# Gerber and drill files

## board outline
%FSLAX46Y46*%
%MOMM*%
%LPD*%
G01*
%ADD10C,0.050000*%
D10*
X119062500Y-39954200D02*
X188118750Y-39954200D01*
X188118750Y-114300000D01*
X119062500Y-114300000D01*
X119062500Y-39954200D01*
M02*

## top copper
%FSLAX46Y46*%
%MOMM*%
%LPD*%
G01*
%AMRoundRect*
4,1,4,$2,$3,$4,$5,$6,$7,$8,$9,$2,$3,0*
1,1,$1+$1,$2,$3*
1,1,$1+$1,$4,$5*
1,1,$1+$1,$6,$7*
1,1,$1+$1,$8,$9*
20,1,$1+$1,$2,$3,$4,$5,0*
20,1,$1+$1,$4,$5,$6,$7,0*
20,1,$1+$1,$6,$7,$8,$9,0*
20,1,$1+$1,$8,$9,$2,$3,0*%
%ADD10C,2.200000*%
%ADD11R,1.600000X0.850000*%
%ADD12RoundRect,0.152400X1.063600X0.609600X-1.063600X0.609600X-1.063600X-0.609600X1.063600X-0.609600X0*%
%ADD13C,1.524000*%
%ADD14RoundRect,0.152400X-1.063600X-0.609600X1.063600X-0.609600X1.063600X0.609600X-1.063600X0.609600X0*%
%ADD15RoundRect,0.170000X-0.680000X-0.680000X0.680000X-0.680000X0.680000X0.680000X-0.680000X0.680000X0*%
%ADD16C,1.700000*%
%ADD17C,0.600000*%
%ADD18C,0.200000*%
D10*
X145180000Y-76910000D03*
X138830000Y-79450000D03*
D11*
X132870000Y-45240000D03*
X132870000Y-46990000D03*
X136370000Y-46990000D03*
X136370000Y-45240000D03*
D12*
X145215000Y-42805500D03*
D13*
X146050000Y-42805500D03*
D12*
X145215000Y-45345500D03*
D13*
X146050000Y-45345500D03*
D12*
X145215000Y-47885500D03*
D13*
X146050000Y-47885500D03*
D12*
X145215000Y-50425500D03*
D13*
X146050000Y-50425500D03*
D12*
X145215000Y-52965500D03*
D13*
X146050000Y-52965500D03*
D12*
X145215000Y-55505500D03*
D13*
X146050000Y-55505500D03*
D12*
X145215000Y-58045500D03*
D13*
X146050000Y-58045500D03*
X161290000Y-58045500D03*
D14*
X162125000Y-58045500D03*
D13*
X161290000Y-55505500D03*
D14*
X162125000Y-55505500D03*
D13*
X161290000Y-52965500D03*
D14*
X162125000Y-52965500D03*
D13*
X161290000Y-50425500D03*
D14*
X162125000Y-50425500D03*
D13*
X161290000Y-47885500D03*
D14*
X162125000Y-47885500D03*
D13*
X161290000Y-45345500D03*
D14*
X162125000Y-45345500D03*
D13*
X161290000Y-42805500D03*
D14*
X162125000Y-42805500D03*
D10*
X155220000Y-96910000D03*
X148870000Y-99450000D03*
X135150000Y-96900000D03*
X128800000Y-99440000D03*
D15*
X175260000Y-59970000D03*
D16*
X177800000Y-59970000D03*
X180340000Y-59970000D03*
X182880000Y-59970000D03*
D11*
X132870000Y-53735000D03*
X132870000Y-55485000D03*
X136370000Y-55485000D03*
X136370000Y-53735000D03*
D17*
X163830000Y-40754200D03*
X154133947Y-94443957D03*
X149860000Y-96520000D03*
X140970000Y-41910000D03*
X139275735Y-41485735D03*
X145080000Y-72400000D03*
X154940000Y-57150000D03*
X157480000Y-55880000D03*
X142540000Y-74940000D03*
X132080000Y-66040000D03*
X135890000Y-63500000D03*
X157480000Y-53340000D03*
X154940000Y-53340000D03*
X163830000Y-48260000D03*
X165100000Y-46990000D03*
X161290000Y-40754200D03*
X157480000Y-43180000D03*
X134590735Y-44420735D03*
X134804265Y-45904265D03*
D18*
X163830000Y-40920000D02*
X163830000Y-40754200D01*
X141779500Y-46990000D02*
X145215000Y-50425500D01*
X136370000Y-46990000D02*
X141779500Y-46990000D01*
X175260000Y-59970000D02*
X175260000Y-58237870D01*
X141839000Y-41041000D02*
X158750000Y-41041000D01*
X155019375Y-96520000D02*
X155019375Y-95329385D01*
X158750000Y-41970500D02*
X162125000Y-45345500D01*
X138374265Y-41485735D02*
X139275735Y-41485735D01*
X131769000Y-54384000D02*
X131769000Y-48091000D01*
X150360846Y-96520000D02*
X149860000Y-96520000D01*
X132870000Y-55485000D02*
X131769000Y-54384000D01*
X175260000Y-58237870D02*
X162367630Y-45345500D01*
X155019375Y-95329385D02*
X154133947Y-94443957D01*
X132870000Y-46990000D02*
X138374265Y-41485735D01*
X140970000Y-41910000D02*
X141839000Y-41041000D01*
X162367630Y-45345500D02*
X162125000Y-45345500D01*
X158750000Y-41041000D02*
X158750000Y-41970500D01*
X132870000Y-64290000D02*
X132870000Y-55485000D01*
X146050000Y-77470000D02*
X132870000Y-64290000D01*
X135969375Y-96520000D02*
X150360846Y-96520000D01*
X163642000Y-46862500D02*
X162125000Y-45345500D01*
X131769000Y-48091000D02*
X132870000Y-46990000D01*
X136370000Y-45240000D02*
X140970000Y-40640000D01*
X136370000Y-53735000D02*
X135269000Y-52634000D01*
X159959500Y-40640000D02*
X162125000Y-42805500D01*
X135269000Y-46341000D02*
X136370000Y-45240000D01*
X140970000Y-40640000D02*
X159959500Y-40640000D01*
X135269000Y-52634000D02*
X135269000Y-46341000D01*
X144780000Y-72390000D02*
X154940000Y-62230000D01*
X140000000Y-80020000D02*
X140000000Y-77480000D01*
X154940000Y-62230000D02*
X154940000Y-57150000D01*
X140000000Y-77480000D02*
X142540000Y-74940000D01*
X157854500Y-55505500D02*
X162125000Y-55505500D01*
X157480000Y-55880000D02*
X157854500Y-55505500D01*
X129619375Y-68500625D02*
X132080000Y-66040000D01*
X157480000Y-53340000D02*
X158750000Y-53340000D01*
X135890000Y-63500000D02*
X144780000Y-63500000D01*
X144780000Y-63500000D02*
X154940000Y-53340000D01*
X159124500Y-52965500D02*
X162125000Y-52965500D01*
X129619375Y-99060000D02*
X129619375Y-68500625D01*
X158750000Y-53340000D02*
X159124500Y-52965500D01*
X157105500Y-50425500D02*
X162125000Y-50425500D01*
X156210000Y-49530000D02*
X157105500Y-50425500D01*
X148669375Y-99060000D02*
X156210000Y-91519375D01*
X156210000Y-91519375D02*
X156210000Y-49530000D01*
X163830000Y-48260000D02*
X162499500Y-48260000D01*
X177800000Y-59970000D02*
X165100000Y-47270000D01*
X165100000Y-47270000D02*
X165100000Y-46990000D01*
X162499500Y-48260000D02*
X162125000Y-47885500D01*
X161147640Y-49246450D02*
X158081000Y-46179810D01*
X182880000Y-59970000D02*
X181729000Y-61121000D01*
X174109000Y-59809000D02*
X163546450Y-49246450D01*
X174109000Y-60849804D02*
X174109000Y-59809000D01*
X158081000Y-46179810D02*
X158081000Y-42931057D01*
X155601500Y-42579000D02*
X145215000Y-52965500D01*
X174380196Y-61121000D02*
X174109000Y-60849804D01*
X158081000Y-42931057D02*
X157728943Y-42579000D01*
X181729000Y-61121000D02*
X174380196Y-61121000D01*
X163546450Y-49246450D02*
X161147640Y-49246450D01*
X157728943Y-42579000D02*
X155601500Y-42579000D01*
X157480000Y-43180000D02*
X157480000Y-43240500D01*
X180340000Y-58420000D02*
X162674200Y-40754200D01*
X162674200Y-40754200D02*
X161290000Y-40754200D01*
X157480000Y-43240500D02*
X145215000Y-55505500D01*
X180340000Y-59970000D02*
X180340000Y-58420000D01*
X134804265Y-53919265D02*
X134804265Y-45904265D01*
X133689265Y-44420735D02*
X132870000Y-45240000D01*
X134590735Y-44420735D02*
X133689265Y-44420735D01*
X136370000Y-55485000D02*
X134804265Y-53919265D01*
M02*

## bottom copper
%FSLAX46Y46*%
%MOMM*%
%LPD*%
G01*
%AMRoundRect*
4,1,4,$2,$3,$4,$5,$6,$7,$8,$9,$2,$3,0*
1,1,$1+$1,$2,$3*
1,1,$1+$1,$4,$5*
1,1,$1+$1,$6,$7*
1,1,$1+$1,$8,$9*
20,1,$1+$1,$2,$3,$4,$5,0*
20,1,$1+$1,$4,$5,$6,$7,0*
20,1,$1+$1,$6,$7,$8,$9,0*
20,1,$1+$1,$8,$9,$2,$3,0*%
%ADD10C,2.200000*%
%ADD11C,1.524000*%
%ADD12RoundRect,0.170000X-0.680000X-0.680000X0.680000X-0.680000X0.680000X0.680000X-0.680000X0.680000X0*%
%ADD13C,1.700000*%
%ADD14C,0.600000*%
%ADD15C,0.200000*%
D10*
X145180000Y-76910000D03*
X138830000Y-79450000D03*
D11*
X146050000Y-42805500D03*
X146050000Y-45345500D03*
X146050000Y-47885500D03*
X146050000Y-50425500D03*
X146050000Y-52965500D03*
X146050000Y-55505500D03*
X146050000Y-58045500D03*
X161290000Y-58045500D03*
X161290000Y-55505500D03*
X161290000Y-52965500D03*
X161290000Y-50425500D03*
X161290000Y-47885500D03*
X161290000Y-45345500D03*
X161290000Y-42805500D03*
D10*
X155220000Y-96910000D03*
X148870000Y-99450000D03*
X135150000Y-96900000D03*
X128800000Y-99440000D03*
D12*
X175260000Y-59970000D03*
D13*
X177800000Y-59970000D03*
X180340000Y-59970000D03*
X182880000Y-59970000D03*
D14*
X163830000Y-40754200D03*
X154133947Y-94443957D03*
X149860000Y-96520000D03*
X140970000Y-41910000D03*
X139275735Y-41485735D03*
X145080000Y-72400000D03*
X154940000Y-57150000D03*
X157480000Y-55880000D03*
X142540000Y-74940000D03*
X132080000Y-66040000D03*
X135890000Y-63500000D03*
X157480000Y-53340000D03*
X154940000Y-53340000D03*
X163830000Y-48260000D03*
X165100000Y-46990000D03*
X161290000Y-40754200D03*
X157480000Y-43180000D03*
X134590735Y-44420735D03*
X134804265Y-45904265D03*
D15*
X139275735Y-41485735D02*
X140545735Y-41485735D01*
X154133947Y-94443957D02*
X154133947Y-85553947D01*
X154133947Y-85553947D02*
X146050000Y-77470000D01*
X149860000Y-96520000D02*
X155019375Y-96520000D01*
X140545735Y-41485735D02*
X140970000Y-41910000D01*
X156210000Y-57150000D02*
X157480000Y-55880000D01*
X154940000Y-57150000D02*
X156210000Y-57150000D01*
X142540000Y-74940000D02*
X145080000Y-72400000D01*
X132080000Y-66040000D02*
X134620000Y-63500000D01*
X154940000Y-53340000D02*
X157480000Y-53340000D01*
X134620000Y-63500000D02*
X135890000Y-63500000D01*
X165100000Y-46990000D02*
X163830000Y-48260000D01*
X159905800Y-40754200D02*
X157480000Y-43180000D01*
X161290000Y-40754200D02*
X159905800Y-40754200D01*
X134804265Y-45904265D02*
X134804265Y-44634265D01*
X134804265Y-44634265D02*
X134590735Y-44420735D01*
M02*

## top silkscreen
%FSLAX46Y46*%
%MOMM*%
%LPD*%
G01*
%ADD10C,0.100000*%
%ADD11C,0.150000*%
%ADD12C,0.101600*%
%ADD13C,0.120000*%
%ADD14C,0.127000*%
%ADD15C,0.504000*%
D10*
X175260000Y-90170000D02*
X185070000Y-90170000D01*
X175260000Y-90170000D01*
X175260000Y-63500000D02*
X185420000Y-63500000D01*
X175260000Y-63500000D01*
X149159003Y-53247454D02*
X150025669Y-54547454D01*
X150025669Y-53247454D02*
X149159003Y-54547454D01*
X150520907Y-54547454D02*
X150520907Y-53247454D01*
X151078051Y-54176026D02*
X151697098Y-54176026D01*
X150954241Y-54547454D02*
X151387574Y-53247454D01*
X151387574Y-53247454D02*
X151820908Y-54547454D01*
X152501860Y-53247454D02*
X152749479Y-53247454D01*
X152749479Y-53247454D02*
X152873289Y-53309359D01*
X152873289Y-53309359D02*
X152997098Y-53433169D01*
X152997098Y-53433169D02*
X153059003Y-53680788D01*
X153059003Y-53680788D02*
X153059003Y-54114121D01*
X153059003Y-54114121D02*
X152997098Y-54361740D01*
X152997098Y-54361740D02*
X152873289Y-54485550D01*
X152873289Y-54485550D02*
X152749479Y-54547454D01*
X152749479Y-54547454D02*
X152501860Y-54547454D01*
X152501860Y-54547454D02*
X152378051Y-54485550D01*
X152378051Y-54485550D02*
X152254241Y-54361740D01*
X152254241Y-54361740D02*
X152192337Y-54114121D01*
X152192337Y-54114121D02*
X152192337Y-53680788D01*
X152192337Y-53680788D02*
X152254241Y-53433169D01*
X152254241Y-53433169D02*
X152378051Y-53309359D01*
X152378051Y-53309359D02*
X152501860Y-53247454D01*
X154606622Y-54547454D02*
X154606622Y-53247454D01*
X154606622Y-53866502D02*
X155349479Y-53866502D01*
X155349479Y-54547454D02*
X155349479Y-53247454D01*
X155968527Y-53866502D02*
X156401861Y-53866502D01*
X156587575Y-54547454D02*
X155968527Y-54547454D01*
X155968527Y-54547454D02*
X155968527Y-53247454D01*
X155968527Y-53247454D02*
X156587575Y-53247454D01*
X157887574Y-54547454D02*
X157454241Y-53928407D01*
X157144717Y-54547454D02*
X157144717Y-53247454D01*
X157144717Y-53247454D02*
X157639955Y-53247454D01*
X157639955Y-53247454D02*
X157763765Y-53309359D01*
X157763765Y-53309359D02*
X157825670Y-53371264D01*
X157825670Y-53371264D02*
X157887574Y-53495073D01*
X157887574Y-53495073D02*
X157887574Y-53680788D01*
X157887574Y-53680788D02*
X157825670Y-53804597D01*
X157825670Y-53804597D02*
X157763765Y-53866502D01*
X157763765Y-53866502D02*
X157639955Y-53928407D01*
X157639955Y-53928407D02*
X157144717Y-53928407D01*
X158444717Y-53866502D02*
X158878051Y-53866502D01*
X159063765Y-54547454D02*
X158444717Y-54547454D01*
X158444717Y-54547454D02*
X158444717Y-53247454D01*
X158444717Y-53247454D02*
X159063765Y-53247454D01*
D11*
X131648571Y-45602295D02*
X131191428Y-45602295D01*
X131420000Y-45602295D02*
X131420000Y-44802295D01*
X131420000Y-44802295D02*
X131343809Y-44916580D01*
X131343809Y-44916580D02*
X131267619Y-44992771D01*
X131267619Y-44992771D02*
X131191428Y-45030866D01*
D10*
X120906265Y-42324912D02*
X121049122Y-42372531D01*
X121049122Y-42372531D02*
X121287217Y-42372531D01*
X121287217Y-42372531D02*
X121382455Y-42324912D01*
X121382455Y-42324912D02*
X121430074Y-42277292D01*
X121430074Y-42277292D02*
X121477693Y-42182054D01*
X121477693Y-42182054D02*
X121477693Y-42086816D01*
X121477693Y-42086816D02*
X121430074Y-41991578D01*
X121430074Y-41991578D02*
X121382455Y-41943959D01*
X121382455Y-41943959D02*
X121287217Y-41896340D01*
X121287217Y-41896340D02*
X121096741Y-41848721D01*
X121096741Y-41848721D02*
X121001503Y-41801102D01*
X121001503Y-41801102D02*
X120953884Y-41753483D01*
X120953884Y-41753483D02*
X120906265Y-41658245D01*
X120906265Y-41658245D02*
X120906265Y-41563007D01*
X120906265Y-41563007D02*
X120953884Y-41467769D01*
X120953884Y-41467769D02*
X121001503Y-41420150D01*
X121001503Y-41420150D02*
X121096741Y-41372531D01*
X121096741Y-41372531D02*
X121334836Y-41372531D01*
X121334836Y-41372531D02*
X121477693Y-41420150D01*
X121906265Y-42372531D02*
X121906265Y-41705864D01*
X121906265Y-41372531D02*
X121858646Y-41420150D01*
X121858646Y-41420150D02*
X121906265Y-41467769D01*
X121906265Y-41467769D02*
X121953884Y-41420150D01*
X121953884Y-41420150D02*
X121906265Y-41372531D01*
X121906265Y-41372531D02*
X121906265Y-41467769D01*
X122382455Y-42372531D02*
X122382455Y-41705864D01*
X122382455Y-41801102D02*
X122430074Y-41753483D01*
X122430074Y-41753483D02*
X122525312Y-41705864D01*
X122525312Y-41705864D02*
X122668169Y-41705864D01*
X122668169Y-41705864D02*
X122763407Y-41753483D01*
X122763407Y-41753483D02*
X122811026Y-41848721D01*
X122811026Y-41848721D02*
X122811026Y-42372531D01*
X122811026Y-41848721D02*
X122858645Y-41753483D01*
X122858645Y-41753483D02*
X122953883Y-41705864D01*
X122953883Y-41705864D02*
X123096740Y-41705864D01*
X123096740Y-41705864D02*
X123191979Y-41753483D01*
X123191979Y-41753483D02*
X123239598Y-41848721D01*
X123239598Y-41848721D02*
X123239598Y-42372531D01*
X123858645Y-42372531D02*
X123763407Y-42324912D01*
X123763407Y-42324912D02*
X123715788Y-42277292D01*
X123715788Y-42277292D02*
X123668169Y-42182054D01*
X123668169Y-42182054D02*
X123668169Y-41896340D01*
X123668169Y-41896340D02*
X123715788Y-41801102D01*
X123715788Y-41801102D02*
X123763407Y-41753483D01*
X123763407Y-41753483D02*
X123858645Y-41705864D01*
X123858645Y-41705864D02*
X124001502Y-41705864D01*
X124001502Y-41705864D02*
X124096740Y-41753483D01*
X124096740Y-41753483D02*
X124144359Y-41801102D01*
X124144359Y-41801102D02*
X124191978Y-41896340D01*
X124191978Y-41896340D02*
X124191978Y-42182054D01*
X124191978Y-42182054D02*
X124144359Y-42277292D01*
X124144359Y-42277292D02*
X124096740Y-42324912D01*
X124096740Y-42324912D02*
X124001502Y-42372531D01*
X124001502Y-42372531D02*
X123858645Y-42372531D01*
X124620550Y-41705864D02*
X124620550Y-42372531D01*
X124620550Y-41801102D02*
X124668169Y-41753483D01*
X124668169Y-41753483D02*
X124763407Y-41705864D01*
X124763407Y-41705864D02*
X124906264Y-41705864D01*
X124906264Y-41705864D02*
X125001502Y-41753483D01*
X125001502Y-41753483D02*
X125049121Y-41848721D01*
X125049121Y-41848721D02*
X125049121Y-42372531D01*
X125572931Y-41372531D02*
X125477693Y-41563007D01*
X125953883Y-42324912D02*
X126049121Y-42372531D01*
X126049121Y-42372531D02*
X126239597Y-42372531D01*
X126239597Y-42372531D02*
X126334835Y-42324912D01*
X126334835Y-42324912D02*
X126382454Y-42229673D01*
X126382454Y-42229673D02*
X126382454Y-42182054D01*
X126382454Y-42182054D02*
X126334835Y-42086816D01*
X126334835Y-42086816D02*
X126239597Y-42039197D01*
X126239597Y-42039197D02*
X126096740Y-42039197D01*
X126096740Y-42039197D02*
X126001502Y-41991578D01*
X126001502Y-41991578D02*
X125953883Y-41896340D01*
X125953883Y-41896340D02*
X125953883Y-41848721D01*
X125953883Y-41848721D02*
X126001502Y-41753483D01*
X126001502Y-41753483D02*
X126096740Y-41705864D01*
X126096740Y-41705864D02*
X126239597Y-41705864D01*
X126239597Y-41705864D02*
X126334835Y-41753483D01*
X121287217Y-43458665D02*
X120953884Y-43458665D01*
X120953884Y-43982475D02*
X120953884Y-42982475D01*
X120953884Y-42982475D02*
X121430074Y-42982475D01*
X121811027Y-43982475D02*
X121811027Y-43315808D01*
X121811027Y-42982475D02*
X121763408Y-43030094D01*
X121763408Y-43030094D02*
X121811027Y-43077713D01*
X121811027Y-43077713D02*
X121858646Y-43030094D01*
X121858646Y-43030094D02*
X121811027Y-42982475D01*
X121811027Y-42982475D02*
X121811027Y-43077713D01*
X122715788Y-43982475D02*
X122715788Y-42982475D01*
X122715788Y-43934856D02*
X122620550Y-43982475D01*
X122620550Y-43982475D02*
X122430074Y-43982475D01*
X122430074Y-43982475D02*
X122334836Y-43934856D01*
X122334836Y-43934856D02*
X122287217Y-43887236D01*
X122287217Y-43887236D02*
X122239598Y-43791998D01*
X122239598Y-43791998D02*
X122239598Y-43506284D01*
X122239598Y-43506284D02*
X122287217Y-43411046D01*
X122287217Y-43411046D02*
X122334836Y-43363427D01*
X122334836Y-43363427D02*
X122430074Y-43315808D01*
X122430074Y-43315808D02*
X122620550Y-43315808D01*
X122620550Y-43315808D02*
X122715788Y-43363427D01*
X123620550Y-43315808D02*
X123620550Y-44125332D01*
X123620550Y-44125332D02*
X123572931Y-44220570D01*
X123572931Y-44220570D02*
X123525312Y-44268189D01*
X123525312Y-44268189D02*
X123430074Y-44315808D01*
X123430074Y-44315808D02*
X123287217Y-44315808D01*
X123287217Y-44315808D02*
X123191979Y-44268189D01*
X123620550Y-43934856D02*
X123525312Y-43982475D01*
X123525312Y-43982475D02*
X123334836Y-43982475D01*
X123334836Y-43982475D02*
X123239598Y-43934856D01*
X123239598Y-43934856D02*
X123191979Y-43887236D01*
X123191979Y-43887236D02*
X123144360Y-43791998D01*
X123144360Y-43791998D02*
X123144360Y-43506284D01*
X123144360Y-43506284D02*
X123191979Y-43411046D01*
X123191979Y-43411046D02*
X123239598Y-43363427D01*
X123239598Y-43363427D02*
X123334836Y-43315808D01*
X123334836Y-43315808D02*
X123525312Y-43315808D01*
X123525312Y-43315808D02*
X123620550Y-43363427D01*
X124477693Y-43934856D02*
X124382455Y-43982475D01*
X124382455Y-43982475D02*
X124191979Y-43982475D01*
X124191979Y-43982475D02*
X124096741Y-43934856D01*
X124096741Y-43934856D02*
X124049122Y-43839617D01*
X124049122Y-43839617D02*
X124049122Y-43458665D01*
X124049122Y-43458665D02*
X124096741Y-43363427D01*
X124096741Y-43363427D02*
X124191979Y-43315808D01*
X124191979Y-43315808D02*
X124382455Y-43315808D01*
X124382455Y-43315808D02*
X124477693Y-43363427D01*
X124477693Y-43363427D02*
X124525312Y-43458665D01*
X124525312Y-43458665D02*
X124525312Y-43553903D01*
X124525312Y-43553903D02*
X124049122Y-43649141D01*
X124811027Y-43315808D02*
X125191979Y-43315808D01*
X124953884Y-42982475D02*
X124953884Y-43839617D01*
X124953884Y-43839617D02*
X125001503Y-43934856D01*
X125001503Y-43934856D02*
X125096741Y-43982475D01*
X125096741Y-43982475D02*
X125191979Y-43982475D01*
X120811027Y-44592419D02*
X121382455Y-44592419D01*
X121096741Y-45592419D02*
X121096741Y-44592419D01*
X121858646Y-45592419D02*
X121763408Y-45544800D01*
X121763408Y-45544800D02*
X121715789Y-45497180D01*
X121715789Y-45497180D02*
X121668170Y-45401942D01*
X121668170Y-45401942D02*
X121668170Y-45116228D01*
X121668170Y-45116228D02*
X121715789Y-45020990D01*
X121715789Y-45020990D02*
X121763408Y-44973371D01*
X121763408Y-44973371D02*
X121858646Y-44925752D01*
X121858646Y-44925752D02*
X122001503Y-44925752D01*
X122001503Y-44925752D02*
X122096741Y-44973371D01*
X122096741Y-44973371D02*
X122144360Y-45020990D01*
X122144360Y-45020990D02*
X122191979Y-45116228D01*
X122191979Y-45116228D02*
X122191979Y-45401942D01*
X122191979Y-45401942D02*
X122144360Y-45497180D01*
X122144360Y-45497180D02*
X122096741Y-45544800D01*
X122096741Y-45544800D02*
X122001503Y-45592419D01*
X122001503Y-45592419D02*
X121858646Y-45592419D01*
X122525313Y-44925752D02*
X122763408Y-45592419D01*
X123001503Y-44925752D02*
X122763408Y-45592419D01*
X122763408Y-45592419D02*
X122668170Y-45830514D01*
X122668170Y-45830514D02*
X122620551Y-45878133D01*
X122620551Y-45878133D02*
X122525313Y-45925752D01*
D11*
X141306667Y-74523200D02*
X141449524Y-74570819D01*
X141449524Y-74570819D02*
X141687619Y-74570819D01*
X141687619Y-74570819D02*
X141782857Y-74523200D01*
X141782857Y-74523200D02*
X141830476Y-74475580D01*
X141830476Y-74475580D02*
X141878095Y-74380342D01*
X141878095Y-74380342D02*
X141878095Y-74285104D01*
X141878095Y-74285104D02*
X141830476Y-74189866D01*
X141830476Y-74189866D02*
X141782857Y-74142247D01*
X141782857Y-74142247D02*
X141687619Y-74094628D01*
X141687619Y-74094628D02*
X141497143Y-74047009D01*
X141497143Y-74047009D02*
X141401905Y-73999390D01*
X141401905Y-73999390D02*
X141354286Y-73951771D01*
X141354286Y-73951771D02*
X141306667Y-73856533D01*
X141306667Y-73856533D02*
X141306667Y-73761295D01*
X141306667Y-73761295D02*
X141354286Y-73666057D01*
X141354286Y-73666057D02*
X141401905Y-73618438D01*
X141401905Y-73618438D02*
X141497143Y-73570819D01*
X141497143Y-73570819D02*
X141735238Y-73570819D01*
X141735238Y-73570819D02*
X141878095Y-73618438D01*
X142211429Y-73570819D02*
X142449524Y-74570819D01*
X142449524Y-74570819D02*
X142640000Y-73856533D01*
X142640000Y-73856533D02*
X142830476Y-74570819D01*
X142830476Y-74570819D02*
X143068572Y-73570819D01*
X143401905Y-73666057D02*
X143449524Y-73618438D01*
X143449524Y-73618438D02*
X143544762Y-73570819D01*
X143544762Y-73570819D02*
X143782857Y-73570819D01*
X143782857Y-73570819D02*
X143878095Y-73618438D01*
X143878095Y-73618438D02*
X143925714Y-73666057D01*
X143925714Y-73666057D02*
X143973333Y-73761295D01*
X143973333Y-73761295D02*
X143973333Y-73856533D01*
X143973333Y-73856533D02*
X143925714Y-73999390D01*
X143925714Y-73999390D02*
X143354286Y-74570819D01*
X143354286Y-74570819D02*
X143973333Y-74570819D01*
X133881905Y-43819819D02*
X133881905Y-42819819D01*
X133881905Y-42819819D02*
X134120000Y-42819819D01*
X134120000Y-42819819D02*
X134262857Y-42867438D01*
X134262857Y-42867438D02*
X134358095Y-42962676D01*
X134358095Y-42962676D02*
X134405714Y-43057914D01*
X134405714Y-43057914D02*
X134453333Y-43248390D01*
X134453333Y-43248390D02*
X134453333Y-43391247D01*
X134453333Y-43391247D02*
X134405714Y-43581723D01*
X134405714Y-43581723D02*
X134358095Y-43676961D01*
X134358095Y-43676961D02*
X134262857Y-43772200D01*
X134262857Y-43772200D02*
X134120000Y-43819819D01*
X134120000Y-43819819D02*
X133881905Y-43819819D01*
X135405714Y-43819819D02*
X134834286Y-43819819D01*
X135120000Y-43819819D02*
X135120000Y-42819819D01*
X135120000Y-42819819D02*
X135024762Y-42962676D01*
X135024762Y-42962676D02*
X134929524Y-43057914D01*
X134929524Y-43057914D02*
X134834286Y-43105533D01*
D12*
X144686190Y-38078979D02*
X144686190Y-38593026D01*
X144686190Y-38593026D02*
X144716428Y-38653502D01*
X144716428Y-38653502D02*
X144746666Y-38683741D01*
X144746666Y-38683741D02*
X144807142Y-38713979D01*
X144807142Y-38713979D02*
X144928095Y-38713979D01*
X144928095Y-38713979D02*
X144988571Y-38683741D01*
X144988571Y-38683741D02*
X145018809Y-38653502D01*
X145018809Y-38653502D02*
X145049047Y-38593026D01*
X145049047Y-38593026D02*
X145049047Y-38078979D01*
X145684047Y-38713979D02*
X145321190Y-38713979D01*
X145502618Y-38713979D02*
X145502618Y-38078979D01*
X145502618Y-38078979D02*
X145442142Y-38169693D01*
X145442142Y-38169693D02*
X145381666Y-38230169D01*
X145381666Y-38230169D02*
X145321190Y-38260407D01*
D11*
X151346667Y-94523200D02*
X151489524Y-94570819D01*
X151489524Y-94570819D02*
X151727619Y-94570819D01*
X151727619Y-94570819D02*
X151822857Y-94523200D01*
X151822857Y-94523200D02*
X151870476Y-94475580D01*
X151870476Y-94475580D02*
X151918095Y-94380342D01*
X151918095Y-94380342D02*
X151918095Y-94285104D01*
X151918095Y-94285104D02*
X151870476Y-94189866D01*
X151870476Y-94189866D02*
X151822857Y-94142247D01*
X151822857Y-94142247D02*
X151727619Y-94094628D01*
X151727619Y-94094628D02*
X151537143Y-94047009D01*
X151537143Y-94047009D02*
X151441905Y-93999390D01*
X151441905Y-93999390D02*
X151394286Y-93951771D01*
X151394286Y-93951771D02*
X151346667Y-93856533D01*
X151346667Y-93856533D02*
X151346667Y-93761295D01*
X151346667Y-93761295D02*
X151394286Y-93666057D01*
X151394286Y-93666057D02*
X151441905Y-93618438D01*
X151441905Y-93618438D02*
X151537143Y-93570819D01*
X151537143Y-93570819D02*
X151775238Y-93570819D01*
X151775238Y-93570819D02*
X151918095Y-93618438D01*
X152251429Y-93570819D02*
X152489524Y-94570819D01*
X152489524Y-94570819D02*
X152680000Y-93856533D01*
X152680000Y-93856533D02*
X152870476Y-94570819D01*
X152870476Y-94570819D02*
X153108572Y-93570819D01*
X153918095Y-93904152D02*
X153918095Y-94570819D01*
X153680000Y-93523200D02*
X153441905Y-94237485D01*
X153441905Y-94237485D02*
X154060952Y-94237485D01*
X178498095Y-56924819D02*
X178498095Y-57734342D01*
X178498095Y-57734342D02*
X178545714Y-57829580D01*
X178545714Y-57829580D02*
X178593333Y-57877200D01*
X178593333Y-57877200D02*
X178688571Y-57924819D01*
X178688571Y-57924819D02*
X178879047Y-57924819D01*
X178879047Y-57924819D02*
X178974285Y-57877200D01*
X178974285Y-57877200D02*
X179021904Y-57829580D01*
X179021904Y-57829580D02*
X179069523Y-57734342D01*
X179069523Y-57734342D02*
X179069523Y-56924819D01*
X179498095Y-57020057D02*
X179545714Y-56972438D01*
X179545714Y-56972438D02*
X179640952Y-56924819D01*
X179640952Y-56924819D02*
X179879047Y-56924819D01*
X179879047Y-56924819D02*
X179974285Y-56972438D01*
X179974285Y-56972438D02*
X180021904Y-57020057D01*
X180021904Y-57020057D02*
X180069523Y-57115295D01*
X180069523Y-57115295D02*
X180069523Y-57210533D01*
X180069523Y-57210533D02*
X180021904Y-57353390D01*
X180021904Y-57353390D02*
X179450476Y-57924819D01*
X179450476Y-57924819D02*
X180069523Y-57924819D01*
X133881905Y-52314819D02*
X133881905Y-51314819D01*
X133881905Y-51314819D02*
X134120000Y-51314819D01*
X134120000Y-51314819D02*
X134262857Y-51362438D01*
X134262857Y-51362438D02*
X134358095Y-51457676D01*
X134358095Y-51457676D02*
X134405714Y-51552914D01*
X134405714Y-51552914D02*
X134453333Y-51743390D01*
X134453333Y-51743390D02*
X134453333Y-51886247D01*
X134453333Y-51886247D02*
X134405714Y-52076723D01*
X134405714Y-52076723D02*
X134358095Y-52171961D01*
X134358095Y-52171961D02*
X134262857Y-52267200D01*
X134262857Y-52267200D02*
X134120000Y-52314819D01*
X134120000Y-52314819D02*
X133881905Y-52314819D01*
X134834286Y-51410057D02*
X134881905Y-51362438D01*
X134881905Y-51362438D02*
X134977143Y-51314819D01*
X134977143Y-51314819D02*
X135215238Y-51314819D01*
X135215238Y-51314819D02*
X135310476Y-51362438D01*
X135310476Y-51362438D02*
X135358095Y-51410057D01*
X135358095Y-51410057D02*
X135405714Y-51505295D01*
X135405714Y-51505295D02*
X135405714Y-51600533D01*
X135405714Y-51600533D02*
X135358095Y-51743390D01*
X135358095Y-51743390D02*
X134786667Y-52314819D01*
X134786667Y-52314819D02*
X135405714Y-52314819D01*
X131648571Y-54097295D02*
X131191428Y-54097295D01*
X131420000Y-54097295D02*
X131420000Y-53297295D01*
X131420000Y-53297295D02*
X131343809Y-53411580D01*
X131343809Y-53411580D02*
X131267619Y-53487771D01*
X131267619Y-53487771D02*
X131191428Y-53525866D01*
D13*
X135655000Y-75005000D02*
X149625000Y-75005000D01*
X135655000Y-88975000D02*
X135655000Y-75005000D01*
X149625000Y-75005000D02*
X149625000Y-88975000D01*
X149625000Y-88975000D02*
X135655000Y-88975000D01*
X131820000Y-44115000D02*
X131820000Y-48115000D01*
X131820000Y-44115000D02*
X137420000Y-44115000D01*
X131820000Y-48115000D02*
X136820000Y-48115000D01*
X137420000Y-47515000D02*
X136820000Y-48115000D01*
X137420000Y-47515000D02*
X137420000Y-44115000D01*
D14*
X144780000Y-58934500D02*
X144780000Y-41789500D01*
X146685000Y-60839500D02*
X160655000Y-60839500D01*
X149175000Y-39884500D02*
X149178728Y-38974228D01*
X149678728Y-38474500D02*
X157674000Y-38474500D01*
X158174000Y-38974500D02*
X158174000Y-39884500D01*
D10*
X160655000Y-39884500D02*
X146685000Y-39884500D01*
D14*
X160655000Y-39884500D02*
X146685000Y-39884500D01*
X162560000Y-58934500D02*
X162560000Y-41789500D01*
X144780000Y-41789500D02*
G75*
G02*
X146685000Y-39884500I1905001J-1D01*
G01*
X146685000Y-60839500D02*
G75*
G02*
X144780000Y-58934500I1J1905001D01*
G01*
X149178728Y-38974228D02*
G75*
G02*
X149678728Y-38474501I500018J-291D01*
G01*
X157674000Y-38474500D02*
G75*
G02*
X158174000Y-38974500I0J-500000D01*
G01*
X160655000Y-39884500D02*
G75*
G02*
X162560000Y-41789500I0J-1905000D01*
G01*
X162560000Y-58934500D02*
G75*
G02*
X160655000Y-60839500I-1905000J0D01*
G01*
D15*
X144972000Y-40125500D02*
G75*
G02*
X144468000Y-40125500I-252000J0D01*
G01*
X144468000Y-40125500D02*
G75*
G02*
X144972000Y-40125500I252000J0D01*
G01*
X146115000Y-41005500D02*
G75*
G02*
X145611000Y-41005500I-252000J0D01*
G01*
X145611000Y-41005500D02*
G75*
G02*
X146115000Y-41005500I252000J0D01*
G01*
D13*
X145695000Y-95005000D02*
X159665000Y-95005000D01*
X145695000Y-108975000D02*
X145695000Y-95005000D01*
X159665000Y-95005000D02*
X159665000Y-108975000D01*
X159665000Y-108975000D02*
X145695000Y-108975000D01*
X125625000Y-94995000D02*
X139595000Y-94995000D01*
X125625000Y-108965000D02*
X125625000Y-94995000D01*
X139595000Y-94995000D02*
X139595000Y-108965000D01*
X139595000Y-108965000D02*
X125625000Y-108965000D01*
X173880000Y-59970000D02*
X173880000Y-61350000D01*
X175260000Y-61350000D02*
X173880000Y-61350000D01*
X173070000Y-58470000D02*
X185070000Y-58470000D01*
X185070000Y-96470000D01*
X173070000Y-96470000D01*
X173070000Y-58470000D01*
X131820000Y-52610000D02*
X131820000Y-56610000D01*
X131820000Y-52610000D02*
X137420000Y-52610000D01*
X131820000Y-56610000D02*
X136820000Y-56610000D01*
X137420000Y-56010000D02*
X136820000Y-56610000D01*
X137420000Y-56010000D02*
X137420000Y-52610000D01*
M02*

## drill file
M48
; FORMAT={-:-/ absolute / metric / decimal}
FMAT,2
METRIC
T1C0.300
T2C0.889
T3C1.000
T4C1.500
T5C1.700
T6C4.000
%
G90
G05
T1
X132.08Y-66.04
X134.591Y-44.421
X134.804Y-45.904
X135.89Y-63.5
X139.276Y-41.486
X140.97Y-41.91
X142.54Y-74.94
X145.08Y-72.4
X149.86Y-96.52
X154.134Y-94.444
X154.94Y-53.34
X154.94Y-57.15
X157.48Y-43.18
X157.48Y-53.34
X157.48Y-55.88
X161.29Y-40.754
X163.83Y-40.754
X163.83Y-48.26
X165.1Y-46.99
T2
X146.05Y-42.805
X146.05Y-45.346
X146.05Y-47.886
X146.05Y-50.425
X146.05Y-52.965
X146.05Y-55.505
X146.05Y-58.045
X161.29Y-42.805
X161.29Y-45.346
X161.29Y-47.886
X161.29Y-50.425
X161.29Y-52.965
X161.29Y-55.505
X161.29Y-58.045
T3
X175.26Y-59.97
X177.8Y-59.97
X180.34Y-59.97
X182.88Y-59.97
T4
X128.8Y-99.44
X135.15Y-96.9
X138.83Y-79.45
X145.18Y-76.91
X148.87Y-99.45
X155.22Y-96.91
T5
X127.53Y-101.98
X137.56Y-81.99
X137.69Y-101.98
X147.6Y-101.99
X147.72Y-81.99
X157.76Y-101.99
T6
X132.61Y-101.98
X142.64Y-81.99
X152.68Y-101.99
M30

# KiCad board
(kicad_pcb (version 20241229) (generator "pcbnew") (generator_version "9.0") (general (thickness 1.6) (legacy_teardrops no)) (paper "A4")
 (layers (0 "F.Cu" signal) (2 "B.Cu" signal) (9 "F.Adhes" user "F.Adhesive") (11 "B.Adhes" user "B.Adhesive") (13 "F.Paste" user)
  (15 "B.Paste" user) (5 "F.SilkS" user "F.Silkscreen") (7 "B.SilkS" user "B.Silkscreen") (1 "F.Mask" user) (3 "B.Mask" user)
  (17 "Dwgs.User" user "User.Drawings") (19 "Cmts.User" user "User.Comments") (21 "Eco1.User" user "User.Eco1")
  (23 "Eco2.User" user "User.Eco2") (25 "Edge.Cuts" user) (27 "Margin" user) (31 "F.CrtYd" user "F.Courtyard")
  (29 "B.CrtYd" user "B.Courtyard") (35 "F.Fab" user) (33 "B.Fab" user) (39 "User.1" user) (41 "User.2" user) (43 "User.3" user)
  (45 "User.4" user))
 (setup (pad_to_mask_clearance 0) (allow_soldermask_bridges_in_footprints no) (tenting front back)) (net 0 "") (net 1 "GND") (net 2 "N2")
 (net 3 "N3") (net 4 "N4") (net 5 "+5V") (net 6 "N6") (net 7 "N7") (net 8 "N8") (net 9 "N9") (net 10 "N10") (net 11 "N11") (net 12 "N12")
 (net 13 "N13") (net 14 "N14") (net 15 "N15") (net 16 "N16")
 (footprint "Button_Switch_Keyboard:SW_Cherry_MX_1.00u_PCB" (layer "F.Cu") (at 145.18 76.91)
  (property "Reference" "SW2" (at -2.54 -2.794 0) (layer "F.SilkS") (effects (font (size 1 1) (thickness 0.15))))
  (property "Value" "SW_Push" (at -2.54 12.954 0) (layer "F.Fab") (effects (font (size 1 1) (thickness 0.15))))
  (fp_line (start -9.525 -1.905) (end 4.445 -1.905) (stroke (width 0.12) (type solid)) (layer "F.SilkS"))
  (fp_line (start -9.525 12.065) (end -9.525 -1.905) (stroke (width 0.12) (type solid)) (layer "F.SilkS"))
  (fp_line (start 4.445 -1.905) (end 4.445 12.065) (stroke (width 0.12) (type solid)) (layer "F.SilkS"))
  (fp_line (start 4.445 12.065) (end -9.525 12.065) (stroke (width 0.12) (type solid)) (layer "F.SilkS"))
  (pad "" np_thru_hole circle (at -7.62 5.08) (size 1.7 1.7) (drill 1.7) (layers "*.Cu" "*.Mask"))
  (pad "" np_thru_hole circle (at -2.54 5.08) (size 4 4) (drill 4) (layers "*.Cu" "*.Mask"))
  (pad "" np_thru_hole circle (at 2.54 5.08) (size 1.7 1.7) (drill 1.7) (layers "*.Cu" "*.Mask"))
  (pad "1" thru_hole circle (at 0 0) (size 2.2 2.2) (drill 1.5) (layers "*.Cu" "*.Mask") (remove_unused_layers no) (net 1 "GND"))
  (pad "2" thru_hole circle (at -6.35 2.54) (size 2.2 2.2) (drill 1.5) (layers "*.Cu" "*.Mask") (remove_unused_layers no) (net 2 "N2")))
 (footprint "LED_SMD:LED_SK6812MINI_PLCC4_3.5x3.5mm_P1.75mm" (layer "F.Cu") (at 134.62 46.115)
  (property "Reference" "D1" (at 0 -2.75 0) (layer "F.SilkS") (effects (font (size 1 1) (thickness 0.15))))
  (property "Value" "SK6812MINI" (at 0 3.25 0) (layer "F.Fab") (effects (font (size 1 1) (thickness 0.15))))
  (fp_line (start -2.8 -2) (end -2.8 2) (stroke (width 0.12) (type default)) (layer "F.SilkS"))
  (fp_line (start -2.8 -2) (end 2.8 -2) (stroke (width 0.12) (type solid)) (layer "F.SilkS"))
  (fp_line (start -2.8 2) (end 2.2 2) (stroke (width 0.12) (type solid)) (layer "F.SilkS"))
  (fp_line (start 2.8 1.4) (end 2.2 2) (stroke (width 0.12) (type default)) (layer "F.SilkS"))
  (fp_line (start 2.8 1.4) (end 2.8 -2) (stroke (width 0.12) (type solid)) (layer "F.SilkS"))
  (pad "1" smd rect (at -1.75 -0.875) (size 1.6 0.85) (layers "F.Cu" "F.Mask" "F.Paste") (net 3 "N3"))
  (pad "2" smd rect (at -1.75 0.875) (size 1.6 0.85) (layers "F.Cu" "F.Mask" "F.Paste") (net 1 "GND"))
  (pad "3" smd rect (at 1.75 0.875) (size 1.6 0.85) (layers "F.Cu" "F.Mask" "F.Paste") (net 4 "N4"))
  (pad "4" smd rect (at 1.75 -0.875) (size 1.6 0.85) (layers "F.Cu" "F.Mask" "F.Paste") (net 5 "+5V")))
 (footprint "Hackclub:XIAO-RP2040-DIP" (layer "F.Cu") (at 153.67 50.4255)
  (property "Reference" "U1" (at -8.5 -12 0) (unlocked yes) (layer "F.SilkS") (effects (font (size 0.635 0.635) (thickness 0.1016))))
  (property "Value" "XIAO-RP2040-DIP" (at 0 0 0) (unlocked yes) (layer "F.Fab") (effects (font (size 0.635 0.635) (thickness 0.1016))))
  (fp_line (start -8.89 8.509) (end -8.89 -8.636) (stroke (width 0.127) (type solid)) (layer "F.SilkS"))
  (fp_line (start -6.985 10.414) (end 6.985 10.414) (stroke (width 0.127) (type solid)) (layer "F.SilkS"))
  (fp_line (start -4.495 -10.541) (end -4.491272 -11.451272) (stroke (width 0.127) (type solid)) (layer "F.SilkS"))
  (fp_line (start -3.991272 -11.951) (end 4.004 -11.951) (stroke (width 0.127) (type solid)) (layer "F.SilkS"))
  (fp_line (start 4.504 -11.451) (end 4.504 -10.541) (stroke (width 0.127) (type solid)) (layer "F.SilkS"))
  (fp_line (start 6.985 -10.541) (end -6.985 -10.541) (stroke (width 0.1) (type solid)) (layer "F.SilkS"))
  (fp_line (start 6.985 -10.541) (end -6.985 -10.541) (stroke (width 0.127) (type solid)) (layer "F.SilkS"))
  (fp_line (start 8.89 8.509) (end 8.89 -8.636) (stroke (width 0.127) (type solid)) (layer "F.SilkS"))
  (fp_arc (start -8.89 -8.636) (mid -8.332038 -9.983038) (end -6.985 -10.541) (stroke (width 0.127) (type solid)) (layer "F.SilkS"))
  (fp_arc (start -6.985 10.414) (mid -8.332038 9.856038) (end -8.89 8.509) (stroke (width 0.127) (type solid)) (layer "F.SilkS"))
  (fp_arc (start -4.491272 -11.451272) (mid -4.344728 -11.80464) (end -3.991272 -11.951) (stroke (width 0.127) (type default))
   (layer "F.SilkS"))
  (fp_arc (start 4.004 -11.951) (mid 4.357553 -11.804553) (end 4.504 -11.451) (stroke (width 0.127) (type default)) (layer "F.SilkS"))
  (fp_arc (start 6.985 -10.541) (mid 8.332038 -9.983038) (end 8.89 -8.636) (stroke (width 0.127) (type solid)) (layer "F.SilkS"))
  (fp_arc (start 8.89 8.509) (mid 8.332038 9.856038) (end 6.985 10.414) (stroke (width 0.127) (type solid)) (layer "F.SilkS"))
  (fp_circle (center -8.95 -10.3) (end -8.95 -10.554) (stroke (width 0.5) (type solid)) (fill yes) (layer "F.SilkS"))
  (fp_circle (center -7.807 -9.42) (end -7.807 -9.674) (stroke (width 0.5) (type solid)) (fill yes) (layer "F.SilkS"))
  (pad "1" smd roundrect (at -8.455 -7.62 180) (size 2.432 1.524) (layers "F.Cu" "F.Mask") (roundrect_rratio 0.1) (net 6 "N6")
   (thermal_bridge_angle 45))
  (pad "1" thru_hole circle (at -7.62 -7.62 180) (size 1.524 1.524) (drill 0.889) (layers "*.Cu" "*.Mask") (remove_unused_layers no)
   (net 6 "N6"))
  (pad "2" smd roundrect (at -8.455 -5.08 180) (size 2.432 1.524) (layers "F.Cu" "F.Mask") (roundrect_rratio 0.1) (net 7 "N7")
   (thermal_bridge_angle 45))
  (pad "2" thru_hole circle (at -7.62 -5.08 180) (size 1.524 1.524) (drill 0.889) (layers "*.Cu" "*.Mask") (remove_unused_layers no)
   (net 7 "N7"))
  (pad "3" smd roundrect (at -8.455 -2.54 180) (size 2.432 1.524) (layers "F.Cu" "F.Mask") (roundrect_rratio 0.1) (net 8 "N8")
   (thermal_bridge_angle 45))
  (pad "3" thru_hole circle (at -7.62 -2.54 180) (size 1.524 1.524) (drill 0.889) (layers "*.Cu" "*.Mask") (remove_unused_layers no)
   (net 8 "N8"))
  (pad "4" smd roundrect (at -8.455 0 180) (size 2.432 1.524) (layers "F.Cu" "F.Mask") (roundrect_rratio 0.1) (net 4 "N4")
   (thermal_bridge_angle 45))
  (pad "4" thru_hole circle (at -7.62 0 180) (size 1.524 1.524) (drill 0.889) (layers "*.Cu" "*.Mask") (remove_unused_layers no)
   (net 4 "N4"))
  (pad "5" smd roundrect (at -8.455 2.54 180) (size 2.432 1.524) (layers "F.Cu" "F.Mask") (roundrect_rratio 0.1) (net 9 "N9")
   (thermal_bridge_angle 45))
  (pad "5" thru_hole circle (at -7.62 2.54 180) (size 1.524 1.524) (drill 0.889) (layers "*.Cu" "*.Mask") (remove_unused_layers no)
   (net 9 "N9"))
  (pad "6" smd roundrect (at -8.455 5.08 180) (size 2.432 1.524) (layers "F.Cu" "F.Mask") (roundrect_rratio 0.1) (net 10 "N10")
   (thermal_bridge_angle 45))
  (pad "6" thru_hole circle (at -7.62 5.08 180) (size 1.524 1.524) (drill 0.889) (layers "*.Cu" "*.Mask") (remove_unused_layers no)
   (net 10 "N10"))
  (pad "7" smd roundrect (at -8.455 7.62 180) (size 2.432 1.524) (layers "F.Cu" "F.Mask") (roundrect_rratio 0.1) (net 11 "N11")
   (thermal_bridge_angle 45))
  (pad "7" thru_hole circle (at -7.62 7.62 180) (size 1.524 1.524) (drill 0.889) (layers "*.Cu" "*.Mask") (remove_unused_layers no)
   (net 11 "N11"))
  (pad "8" thru_hole circle (at 7.62 7.62) (size 1.524 1.524) (drill 0.889) (layers "*.Cu" "*.Mask") (remove_unused_layers no)
   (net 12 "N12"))
  (pad "8" smd roundrect (at 8.455 7.62) (size 2.432 1.524) (layers "F.Cu" "F.Mask") (roundrect_rratio 0.1) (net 12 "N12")
   (thermal_bridge_angle 45))
  (pad "9" thru_hole circle (at 7.62 5.08) (size 1.524 1.524) (drill 0.889) (layers "*.Cu" "*.Mask") (remove_unused_layers no) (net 2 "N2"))
  (pad "9" smd roundrect (at 8.455 5.08) (size 2.432 1.524) (layers "F.Cu" "F.Mask") (roundrect_rratio 0.1) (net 2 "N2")
   (thermal_bridge_angle 45))
  (pad "10" thru_hole circle (at 7.62 2.54) (size 1.524 1.524) (drill 0.889) (layers "*.Cu" "*.Mask") (remove_unused_layers no)
   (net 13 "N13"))
  (pad "10" smd roundrect (at 8.455 2.54) (size 2.432 1.524) (layers "F.Cu" "F.Mask") (roundrect_rratio 0.1) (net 13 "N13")
   (thermal_bridge_angle 45))
  (pad "11" thru_hole circle (at 7.62 0) (size 1.524 1.524) (drill 0.889) (layers "*.Cu" "*.Mask") (remove_unused_layers no) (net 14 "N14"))
  (pad "11" smd roundrect (at 8.455 0) (size 2.432 1.524) (layers "F.Cu" "F.Mask") (roundrect_rratio 0.1) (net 14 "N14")
   (thermal_bridge_angle 45))
  (pad "12" thru_hole circle (at 7.62 -2.54) (size 1.524 1.524) (drill 0.889) (layers "*.Cu" "*.Mask") (remove_unused_layers no)
   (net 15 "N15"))
  (pad "12" smd roundrect (at 8.455 -2.54) (size 2.432 1.524) (layers "F.Cu" "F.Mask") (roundrect_rratio 0.1) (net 15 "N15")
   (thermal_bridge_angle 45))
  (pad "13" thru_hole circle (at 7.62 -5.08) (size 1.524 1.524) (drill 0.889) (layers "*.Cu" "*.Mask") (remove_unused_layers no)
   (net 1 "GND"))
  (pad "13" smd roundrect (at 8.455 -5.08) (size 2.432 1.524) (layers "F.Cu" "F.Mask") (roundrect_rratio 0.1) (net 1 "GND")
   (thermal_bridge_angle 45))
  (pad "14" thru_hole circle (at 7.62 -7.62) (size 1.524 1.524) (drill 0.889) (layers "*.Cu" "*.Mask") (remove_unused_layers no)
   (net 5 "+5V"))
  (pad "14" smd roundrect (at 8.455 -7.62) (size 2.432 1.524) (layers "F.Cu" "F.Mask") (roundrect_rratio 0.1) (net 5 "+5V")
   (thermal_bridge_angle 45)))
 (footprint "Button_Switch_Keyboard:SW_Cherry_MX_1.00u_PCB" (layer "F.Cu") (at 155.22 96.91)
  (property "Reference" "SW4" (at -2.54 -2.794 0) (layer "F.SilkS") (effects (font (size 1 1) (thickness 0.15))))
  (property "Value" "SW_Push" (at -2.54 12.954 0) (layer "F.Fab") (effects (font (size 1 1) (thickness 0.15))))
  (fp_line (start -9.525 -1.905) (end 4.445 -1.905) (stroke (width 0.12) (type solid)) (layer "F.SilkS"))
  (fp_line (start -9.525 12.065) (end -9.525 -1.905) (stroke (width 0.12) (type solid)) (layer "F.SilkS"))
  (fp_line (start 4.445 -1.905) (end 4.445 12.065) (stroke (width 0.12) (type solid)) (layer "F.SilkS"))
  (fp_line (start 4.445 12.065) (end -9.525 12.065) (stroke (width 0.12) (type solid)) (layer "F.SilkS"))
  (pad "" np_thru_hole circle (at -7.62 5.08) (size 1.7 1.7) (drill 1.7) (layers "*.Cu" "*.Mask"))
  (pad "" np_thru_hole circle (at -2.54 5.08) (size 4 4) (drill 4) (layers "*.Cu" "*.Mask"))
  (pad "" np_thru_hole circle (at 2.54 5.08) (size 1.7 1.7) (drill 1.7) (layers "*.Cu" "*.Mask"))
  (pad "1" thru_hole circle (at 0 0) (size 2.2 2.2) (drill 1.5) (layers "*.Cu" "*.Mask") (remove_unused_layers no) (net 1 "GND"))
  (pad "2" thru_hole circle (at -6.35 2.54) (size 2.2 2.2) (drill 1.5) (layers "*.Cu" "*.Mask") (remove_unused_layers no) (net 14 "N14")))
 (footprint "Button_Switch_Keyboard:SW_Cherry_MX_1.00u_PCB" (layer "F.Cu") (at 135.15 96.9)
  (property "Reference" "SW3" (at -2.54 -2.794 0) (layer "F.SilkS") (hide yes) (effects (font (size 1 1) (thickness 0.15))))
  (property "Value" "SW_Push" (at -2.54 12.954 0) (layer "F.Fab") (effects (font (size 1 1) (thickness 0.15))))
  (fp_line (start -9.525 -1.905) (end 4.445 -1.905) (stroke (width 0.12) (type solid)) (layer "F.SilkS"))
  (fp_line (start -9.525 12.065) (end -9.525 -1.905) (stroke (width 0.12) (type solid)) (layer "F.SilkS"))
  (fp_line (start 4.445 -1.905) (end 4.445 12.065) (stroke (width 0.12) (type solid)) (layer "F.SilkS"))
  (fp_line (start 4.445 12.065) (end -9.525 12.065) (stroke (width 0.12) (type solid)) (layer "F.SilkS"))
  (pad "" np_thru_hole circle (at -7.62 5.08) (size 1.7 1.7) (drill 1.7) (layers "*.Cu" "*.Mask"))
  (pad "" np_thru_hole circle (at -2.54 5.08) (size 4 4) (drill 4) (layers "*.Cu" "*.Mask"))
  (pad "" np_thru_hole circle (at 2.54 5.08) (size 1.7 1.7) (drill 1.7) (layers "*.Cu" "*.Mask"))
  (pad "1" thru_hole circle (at 0 0) (size 2.2 2.2) (drill 1.5) (layers "*.Cu" "*.Mask") (remove_unused_layers no) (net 1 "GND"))
  (pad "2" thru_hole circle (at -6.35 2.54) (size 2.2 2.2) (drill 1.5) (layers "*.Cu" "*.Mask") (remove_unused_layers no) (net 13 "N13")))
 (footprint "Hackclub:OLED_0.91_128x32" (layer "F.Cu") (at 175.26 59.97)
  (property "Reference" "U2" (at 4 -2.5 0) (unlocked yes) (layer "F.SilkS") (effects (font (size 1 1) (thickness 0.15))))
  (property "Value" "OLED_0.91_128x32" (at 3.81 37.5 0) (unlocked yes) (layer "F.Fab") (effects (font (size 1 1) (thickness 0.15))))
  (fp_line (start -1.38 0) (end -1.38 1.38) (stroke (width 0.12) (type solid)) (layer "F.SilkS"))
  (fp_line (start 0 1.38) (end -1.38 1.38) (stroke (width 0.12) (type solid)) (layer "F.SilkS"))
  (fp_rect (start -2.19 -1.5) (end 9.81 36.5) (stroke (width 0.12) (type solid)) (fill no) (layer "F.SilkS"))
  (pad "1" thru_hole roundrect (at 0 0) (size 1.7 1.7) (drill 1) (layers "*.Cu" "*.Mask") (remove_unused_layers no) (roundrect_rratio 0.1)
   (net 1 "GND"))
  (pad "2" thru_hole circle (at 2.54 0) (size 1.7 1.7) (drill 1) (layers "*.Cu" "*.Mask") (remove_unused_layers no) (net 15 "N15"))
  (pad "3" thru_hole circle (at 5.08 0) (size 1.7 1.7) (drill 1) (layers "*.Cu" "*.Mask") (remove_unused_layers no) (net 10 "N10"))
  (pad "4" thru_hole circle (at 7.62 0) (size 1.7 1.7) (drill 1) (layers "*.Cu" "*.Mask") (remove_unused_layers no) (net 9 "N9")))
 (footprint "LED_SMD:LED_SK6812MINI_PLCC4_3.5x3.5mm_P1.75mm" (layer "F.Cu") (at 134.62 54.61)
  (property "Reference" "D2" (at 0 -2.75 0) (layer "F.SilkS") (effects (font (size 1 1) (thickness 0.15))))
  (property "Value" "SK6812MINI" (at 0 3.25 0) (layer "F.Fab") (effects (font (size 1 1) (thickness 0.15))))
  (fp_line (start -2.8 -2) (end -2.8 2) (stroke (width 0.12) (type default)) (layer "F.SilkS"))
  (fp_line (start -2.8 -2) (end 2.8 -2) (stroke (width 0.12) (type solid)) (layer "F.SilkS"))
  (fp_line (start -2.8 2) (end 2.2 2) (stroke (width 0.12) (type solid)) (layer "F.SilkS"))
  (fp_line (start 2.8 1.4) (end 2.2 2) (stroke (width 0.12) (type default)) (layer "F.SilkS"))
  (fp_line (start 2.8 1.4) (end 2.8 -2) (stroke (width 0.12) (type solid)) (layer "F.SilkS"))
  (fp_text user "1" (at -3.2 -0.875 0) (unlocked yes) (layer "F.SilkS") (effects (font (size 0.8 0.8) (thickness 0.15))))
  (pad "1" smd rect (at -1.75 -0.875) (size 1.6 0.85) (layers "F.Cu" "F.Mask" "F.Paste") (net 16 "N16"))
  (pad "2" smd rect (at -1.75 0.875) (size 1.6 0.85) (layers "F.Cu" "F.Mask" "F.Paste") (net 1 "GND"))
  (pad "3" smd rect (at 1.75 0.875) (size 1.6 0.85) (layers "F.Cu" "F.Mask" "F.Paste") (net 3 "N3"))
  (pad "4" smd rect (at 1.75 -0.875) (size 1.6 0.85) (layers "F.Cu" "F.Mask" "F.Paste") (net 5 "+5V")))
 (gr_rect (start 175.26 90.17) (end 185.07 90.17) (stroke (width 0.1) (type default)) (fill no) (layer "F.SilkS"))
 (gr_rect (start 175.26 63.5) (end 185.42 63.5) (stroke (width 0.1) (type default)) (fill no) (layer "F.SilkS"))
 (gr_rect (start 119.0625 39.9542) (end 188.11875 114.3) (stroke (width 0.05) (type default)) (fill no) (layer "Edge.Cuts"))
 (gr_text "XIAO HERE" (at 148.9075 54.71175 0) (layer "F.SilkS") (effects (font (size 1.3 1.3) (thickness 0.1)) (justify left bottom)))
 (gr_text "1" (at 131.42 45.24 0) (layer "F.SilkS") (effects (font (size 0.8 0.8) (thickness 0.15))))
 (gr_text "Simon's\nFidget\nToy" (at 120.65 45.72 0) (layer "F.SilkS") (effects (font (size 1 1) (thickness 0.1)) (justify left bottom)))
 (segment (start 163.83 40.92) (end 163.83 40.7542) (width 0.2) (layer "F.Cu") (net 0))
 (via (at 163.83 40.7542) (size 0.6) (drill 0.3) (layers "F.Cu" "B.Cu") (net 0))
 (segment (start 141.7795 46.99) (end 145.215 50.4255) (width 0.2) (layer "F.Cu") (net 4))
 (segment (start 136.37 46.99) (end 141.7795 46.99) (width 0.2) (layer "F.Cu") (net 4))
 (segment (start 175.26 59.97) (end 175.26 58.23787) (width 0.2) (layer "F.Cu") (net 1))
 (segment (start 141.839 41.041) (end 158.75 41.041) (width 0.2) (layer "F.Cu") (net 1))
 (segment (start 155.019375 96.52) (end 155.019375 95.329385) (width 0.2) (layer "F.Cu") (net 1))
 (segment (start 158.75 41.9705) (end 162.125 45.3455) (width 0.2) (layer "F.Cu") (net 1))
 (segment (start 138.374265 41.485735) (end 139.275735 41.485735) (width 0.2) (layer "F.Cu") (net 1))
 (segment (start 131.769 54.384) (end 131.769 48.091) (width 0.2) (layer "F.Cu") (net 1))
 (segment (start 150.360846 96.52) (end 149.86 96.52) (width 0.2) (layer "F.Cu") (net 1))
 (segment (start 132.87 55.485) (end 131.769 54.384) (width 0.2) (layer "F.Cu") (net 1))
 (segment (start 175.26 58.23787) (end 162.36763 45.3455) (width 0.2) (layer "F.Cu") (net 1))
 (segment (start 155.019375 95.329385) (end 154.133947 94.443957) (width 0.2) (layer "F.Cu") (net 1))
 (segment (start 132.87 46.99) (end 138.374265 41.485735) (width 0.2) (layer "F.Cu") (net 1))
 (segment (start 140.97 41.91) (end 141.839 41.041) (width 0.2) (layer "F.Cu") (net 1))
 (segment (start 162.36763 45.3455) (end 162.125 45.3455) (width 0.2) (layer "F.Cu") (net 1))
 (segment (start 158.75 41.041) (end 158.75 41.9705) (width 0.2) (layer "F.Cu") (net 1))
 (segment (start 132.87 64.29) (end 132.87 55.485) (width 0.2) (layer "F.Cu") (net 1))
 (segment (start 146.05 77.47) (end 132.87 64.29) (width 0.2) (layer "F.Cu") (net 1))
 (segment (start 135.969375 96.52) (end 150.360846 96.52) (width 0.2) (layer "F.Cu") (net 1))
 (segment (start 163.642 46.8625) (end 162.125 45.3455) (width 0.2) (layer "F.Cu") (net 1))
 (segment (start 131.769 48.091) (end 132.87 46.99) (width 0.2) (layer "F.Cu") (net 1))
 (via (at 154.133947 94.443957) (size 0.6) (drill 0.3) (layers "F.Cu" "B.Cu") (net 1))
 (via (at 149.86 96.52) (size 0.6) (drill 0.3) (layers "F.Cu" "B.Cu") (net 1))
 (via (at 140.97 41.91) (size 0.6) (drill 0.3) (layers "F.Cu" "B.Cu") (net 1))
 (via (at 139.275735 41.485735) (size 0.6) (drill 0.3) (layers "F.Cu" "B.Cu") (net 1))
 (segment (start 139.275735 41.485735) (end 140.545735 41.485735) (width 0.2) (layer "B.Cu") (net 1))
 (segment (start 154.133947 94.443957) (end 154.133947 85.553947) (width 0.2) (layer "B.Cu") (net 1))
 (segment (start 154.133947 85.553947) (end 146.05 77.47) (width 0.2) (layer "B.Cu") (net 1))
 (segment (start 149.86 96.52) (end 155.019375 96.52) (width 0.2) (layer "B.Cu") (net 1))
 (segment (start 140.545735 41.485735) (end 140.97 41.91) (width 0.2) (layer "B.Cu") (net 1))
 (segment (start 136.37 45.24) (end 140.97 40.64) (width 0.2) (layer "F.Cu") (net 5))
 (segment (start 136.37 53.735) (end 135.269 52.634) (width 0.2) (layer "F.Cu") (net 5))
 (segment (start 159.9595 40.64) (end 162.125 42.8055) (width 0.2) (layer "F.Cu") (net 5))
 (segment (start 135.269 46.341) (end 136.37 45.24) (width 0.2) (layer "F.Cu") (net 5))
 (segment (start 140.97 40.64) (end 159.9595 40.64) (width 0.2) (layer "F.Cu") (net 5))
 (segment (start 135.269 52.634) (end 135.269 46.341) (width 0.2) (layer "F.Cu") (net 5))
 (segment (start 144.78 72.39) (end 154.94 62.23) (width 0.2) (layer "F.Cu") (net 2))
 (segment (start 140 80.02) (end 140 77.48) (width 0.2) (layer "F.Cu") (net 2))
 (segment (start 154.94 62.23) (end 154.94 57.15) (width 0.2) (layer "F.Cu") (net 2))
 (segment (start 140 77.48) (end 142.54 74.94) (width 0.2) (layer "F.Cu") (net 2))
 (segment (start 157.8545 55.5055) (end 162.125 55.5055) (width 0.2) (layer "F.Cu") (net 2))
 (segment (start 157.48 55.88) (end 157.8545 55.5055) (width 0.2) (layer "F.Cu") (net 2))
 (via (at 145.08 72.4) (size 0.6) (drill 0.3) (layers "F.Cu" "B.Cu") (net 2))
 (via (at 154.94 57.15) (size 0.6) (drill 0.3) (layers "F.Cu" "B.Cu") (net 2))
 (via (at 157.48 55.88) (size 0.6) (drill 0.3) (layers "F.Cu" "B.Cu") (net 2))
 (via (at 142.54 74.94) (size 0.6) (drill 0.3) (layers "F.Cu" "B.Cu") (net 2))
 (segment (start 156.21 57.15) (end 157.48 55.88) (width 0.2) (layer "B.Cu") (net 2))
 (segment (start 154.94 57.15) (end 156.21 57.15) (width 0.2) (layer "B.Cu") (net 2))
 (segment (start 142.54 74.94) (end 145.08 72.4) (width 0.2) (layer "B.Cu") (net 2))
 (segment (start 129.619375 68.500625) (end 132.08 66.04) (width 0.2) (layer "F.Cu") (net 13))
 (segment (start 157.48 53.34) (end 158.75 53.34) (width 0.2) (layer "F.Cu") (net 13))
 (segment (start 135.89 63.5) (end 144.78 63.5) (width 0.2) (layer "F.Cu") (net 13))
 (segment (start 144.78 63.5) (end 154.94 53.34) (width 0.2) (layer "F.Cu") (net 13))
 (segment (start 159.1245 52.9655) (end 162.125 52.9655) (width 0.2) (layer "F.Cu") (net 13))
 (segment (start 129.619375 99.06) (end 129.619375 68.500625) (width 0.2) (layer "F.Cu") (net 13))
 (segment (start 158.75 53.34) (end 159.1245 52.9655) (width 0.2) (layer "F.Cu") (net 13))
 (via (at 132.08 66.04) (size 0.6) (drill 0.3) (layers "F.Cu" "B.Cu") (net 13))
 (via (at 135.89 63.5) (size 0.6) (drill 0.3) (layers "F.Cu" "B.Cu") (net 13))
 (via (at 157.48 53.34) (size 0.6) (drill 0.3) (layers "F.Cu" "B.Cu") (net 13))
 (via (at 154.94 53.34) (size 0.6) (drill 0.3) (layers "F.Cu" "B.Cu") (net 13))
 (segment (start 132.08 66.04) (end 134.62 63.5) (width 0.2) (layer "B.Cu") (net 13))
 (segment (start 154.94 53.34) (end 157.48 53.34) (width 0.2) (layer "B.Cu") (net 13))
 (segment (start 134.62 63.5) (end 135.89 63.5) (width 0.2) (layer "B.Cu") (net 13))
 (segment (start 157.1055 50.4255) (end 162.125 50.4255) (width 0.2) (layer "F.Cu") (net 14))
 (segment (start 156.21 49.53) (end 157.1055 50.4255) (width 0.2) (layer "F.Cu") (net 14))
 (segment (start 148.669375 99.06) (end 156.21 91.519375) (width 0.2) (layer "F.Cu") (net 14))
 (segment (start 156.21 91.519375) (end 156.21 49.53) (width 0.2) (layer "F.Cu") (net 14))
 (segment (start 163.83 48.26) (end 162.4995 48.26) (width 0.2) (layer "F.Cu") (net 15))
 (segment (start 177.8 59.97) (end 165.1 47.27) (width 0.2) (layer "F.Cu") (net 15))
 (segment (start 165.1 47.27) (end 165.1 46.99) (width 0.2) (layer "F.Cu") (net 15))
 (segment (start 162.4995 48.26) (end 162.125 47.8855) (width 0.2) (layer "F.Cu") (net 15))
 (via (at 163.83 48.26) (size 0.6) (drill 0.3) (layers "F.Cu" "B.Cu") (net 15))
 (via (at 165.1 46.99) (size 0.6) (drill 0.3) (layers "F.Cu" "B.Cu") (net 15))
 (segment (start 165.1 46.99) (end 163.83 48.26) (width 0.2) (layer "B.Cu") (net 15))
 (segment (start 161.14764 49.24645) (end 158.081 46.17981) (width 0.2) (layer "F.Cu") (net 9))
 (segment (start 182.88 59.97) (end 181.729 61.121) (width 0.2) (layer "F.Cu") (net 9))
 (segment (start 174.109 59.809) (end 163.54645 49.24645) (width 0.2) (layer "F.Cu") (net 9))
 (segment (start 174.109 60.849804) (end 174.109 59.809) (width 0.2) (layer "F.Cu") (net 9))
 (segment (start 158.081 46.17981) (end 158.081 42.931057) (width 0.2) (layer "F.Cu") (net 9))
 (segment (start 155.6015 42.579) (end 145.215 52.9655) (width 0.2) (layer "F.Cu") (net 9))
 (segment (start 174.380196 61.121) (end 174.109 60.849804) (width 0.2) (layer "F.Cu") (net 9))
 (segment (start 158.081 42.931057) (end 157.728943 42.579) (width 0.2) (layer "F.Cu") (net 9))
 (segment (start 181.729 61.121) (end 174.380196 61.121) (width 0.2) (layer "F.Cu") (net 9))
 (segment (start 163.54645 49.24645) (end 161.14764 49.24645) (width 0.2) (layer "F.Cu") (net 9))
 (segment (start 157.728943 42.579) (end 155.6015 42.579) (width 0.2) (layer "F.Cu") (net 9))
 (segment (start 157.48 43.18) (end 157.48 43.2405) (width 0.2) (layer "F.Cu") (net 10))
 (segment (start 180.34 58.42) (end 162.6742 40.7542) (width 0.2) (layer "F.Cu") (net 10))
 (segment (start 162.6742 40.7542) (end 161.29 40.7542) (width 0.2) (layer "F.Cu") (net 10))
 (segment (start 157.48 43.2405) (end 145.215 55.5055) (width 0.2) (layer "F.Cu") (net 10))
 (segment (start 180.34 59.97) (end 180.34 58.42) (width 0.2) (layer "F.Cu") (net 10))
 (via (at 161.29 40.7542) (size 0.6) (drill 0.3) (layers "F.Cu" "B.Cu") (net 10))
 (via (at 157.48 43.18) (size 0.6) (drill 0.3) (layers "F.Cu" "B.Cu") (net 10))
 (segment (start 159.9058 40.7542) (end 157.48 43.18) (width 0.2) (layer "B.Cu") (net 10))
 (segment (start 161.29 40.7542) (end 159.9058 40.7542) (width 0.2) (layer "B.Cu") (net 10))
 (segment (start 134.804265 53.919265) (end 134.804265 45.904265) (width 0.2) (layer "F.Cu") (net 3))
 (segment (start 133.689265 44.420735) (end 132.87 45.24) (width 0.2) (layer "F.Cu") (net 3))
 (segment (start 134.590735 44.420735) (end 133.689265 44.420735) (width 0.2) (layer "F.Cu") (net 3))
 (segment (start 136.37 55.485) (end 134.804265 53.919265) (width 0.2) (layer "F.Cu") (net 3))
 (via (at 134.590735 44.420735) (size 0.6) (drill 0.3) (layers "F.Cu" "B.Cu") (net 3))
 (via (at 134.804265 45.904265) (size 0.6) (drill 0.3) (layers "F.Cu" "B.Cu") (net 3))
 (segment (start 134.804265 45.904265) (end 134.804265 44.634265) (width 0.2) (layer "B.Cu") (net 3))
 (segment (start 134.804265 44.634265) (end 134.590735 44.420735) (width 0.2) (layer "B.Cu") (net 3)))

